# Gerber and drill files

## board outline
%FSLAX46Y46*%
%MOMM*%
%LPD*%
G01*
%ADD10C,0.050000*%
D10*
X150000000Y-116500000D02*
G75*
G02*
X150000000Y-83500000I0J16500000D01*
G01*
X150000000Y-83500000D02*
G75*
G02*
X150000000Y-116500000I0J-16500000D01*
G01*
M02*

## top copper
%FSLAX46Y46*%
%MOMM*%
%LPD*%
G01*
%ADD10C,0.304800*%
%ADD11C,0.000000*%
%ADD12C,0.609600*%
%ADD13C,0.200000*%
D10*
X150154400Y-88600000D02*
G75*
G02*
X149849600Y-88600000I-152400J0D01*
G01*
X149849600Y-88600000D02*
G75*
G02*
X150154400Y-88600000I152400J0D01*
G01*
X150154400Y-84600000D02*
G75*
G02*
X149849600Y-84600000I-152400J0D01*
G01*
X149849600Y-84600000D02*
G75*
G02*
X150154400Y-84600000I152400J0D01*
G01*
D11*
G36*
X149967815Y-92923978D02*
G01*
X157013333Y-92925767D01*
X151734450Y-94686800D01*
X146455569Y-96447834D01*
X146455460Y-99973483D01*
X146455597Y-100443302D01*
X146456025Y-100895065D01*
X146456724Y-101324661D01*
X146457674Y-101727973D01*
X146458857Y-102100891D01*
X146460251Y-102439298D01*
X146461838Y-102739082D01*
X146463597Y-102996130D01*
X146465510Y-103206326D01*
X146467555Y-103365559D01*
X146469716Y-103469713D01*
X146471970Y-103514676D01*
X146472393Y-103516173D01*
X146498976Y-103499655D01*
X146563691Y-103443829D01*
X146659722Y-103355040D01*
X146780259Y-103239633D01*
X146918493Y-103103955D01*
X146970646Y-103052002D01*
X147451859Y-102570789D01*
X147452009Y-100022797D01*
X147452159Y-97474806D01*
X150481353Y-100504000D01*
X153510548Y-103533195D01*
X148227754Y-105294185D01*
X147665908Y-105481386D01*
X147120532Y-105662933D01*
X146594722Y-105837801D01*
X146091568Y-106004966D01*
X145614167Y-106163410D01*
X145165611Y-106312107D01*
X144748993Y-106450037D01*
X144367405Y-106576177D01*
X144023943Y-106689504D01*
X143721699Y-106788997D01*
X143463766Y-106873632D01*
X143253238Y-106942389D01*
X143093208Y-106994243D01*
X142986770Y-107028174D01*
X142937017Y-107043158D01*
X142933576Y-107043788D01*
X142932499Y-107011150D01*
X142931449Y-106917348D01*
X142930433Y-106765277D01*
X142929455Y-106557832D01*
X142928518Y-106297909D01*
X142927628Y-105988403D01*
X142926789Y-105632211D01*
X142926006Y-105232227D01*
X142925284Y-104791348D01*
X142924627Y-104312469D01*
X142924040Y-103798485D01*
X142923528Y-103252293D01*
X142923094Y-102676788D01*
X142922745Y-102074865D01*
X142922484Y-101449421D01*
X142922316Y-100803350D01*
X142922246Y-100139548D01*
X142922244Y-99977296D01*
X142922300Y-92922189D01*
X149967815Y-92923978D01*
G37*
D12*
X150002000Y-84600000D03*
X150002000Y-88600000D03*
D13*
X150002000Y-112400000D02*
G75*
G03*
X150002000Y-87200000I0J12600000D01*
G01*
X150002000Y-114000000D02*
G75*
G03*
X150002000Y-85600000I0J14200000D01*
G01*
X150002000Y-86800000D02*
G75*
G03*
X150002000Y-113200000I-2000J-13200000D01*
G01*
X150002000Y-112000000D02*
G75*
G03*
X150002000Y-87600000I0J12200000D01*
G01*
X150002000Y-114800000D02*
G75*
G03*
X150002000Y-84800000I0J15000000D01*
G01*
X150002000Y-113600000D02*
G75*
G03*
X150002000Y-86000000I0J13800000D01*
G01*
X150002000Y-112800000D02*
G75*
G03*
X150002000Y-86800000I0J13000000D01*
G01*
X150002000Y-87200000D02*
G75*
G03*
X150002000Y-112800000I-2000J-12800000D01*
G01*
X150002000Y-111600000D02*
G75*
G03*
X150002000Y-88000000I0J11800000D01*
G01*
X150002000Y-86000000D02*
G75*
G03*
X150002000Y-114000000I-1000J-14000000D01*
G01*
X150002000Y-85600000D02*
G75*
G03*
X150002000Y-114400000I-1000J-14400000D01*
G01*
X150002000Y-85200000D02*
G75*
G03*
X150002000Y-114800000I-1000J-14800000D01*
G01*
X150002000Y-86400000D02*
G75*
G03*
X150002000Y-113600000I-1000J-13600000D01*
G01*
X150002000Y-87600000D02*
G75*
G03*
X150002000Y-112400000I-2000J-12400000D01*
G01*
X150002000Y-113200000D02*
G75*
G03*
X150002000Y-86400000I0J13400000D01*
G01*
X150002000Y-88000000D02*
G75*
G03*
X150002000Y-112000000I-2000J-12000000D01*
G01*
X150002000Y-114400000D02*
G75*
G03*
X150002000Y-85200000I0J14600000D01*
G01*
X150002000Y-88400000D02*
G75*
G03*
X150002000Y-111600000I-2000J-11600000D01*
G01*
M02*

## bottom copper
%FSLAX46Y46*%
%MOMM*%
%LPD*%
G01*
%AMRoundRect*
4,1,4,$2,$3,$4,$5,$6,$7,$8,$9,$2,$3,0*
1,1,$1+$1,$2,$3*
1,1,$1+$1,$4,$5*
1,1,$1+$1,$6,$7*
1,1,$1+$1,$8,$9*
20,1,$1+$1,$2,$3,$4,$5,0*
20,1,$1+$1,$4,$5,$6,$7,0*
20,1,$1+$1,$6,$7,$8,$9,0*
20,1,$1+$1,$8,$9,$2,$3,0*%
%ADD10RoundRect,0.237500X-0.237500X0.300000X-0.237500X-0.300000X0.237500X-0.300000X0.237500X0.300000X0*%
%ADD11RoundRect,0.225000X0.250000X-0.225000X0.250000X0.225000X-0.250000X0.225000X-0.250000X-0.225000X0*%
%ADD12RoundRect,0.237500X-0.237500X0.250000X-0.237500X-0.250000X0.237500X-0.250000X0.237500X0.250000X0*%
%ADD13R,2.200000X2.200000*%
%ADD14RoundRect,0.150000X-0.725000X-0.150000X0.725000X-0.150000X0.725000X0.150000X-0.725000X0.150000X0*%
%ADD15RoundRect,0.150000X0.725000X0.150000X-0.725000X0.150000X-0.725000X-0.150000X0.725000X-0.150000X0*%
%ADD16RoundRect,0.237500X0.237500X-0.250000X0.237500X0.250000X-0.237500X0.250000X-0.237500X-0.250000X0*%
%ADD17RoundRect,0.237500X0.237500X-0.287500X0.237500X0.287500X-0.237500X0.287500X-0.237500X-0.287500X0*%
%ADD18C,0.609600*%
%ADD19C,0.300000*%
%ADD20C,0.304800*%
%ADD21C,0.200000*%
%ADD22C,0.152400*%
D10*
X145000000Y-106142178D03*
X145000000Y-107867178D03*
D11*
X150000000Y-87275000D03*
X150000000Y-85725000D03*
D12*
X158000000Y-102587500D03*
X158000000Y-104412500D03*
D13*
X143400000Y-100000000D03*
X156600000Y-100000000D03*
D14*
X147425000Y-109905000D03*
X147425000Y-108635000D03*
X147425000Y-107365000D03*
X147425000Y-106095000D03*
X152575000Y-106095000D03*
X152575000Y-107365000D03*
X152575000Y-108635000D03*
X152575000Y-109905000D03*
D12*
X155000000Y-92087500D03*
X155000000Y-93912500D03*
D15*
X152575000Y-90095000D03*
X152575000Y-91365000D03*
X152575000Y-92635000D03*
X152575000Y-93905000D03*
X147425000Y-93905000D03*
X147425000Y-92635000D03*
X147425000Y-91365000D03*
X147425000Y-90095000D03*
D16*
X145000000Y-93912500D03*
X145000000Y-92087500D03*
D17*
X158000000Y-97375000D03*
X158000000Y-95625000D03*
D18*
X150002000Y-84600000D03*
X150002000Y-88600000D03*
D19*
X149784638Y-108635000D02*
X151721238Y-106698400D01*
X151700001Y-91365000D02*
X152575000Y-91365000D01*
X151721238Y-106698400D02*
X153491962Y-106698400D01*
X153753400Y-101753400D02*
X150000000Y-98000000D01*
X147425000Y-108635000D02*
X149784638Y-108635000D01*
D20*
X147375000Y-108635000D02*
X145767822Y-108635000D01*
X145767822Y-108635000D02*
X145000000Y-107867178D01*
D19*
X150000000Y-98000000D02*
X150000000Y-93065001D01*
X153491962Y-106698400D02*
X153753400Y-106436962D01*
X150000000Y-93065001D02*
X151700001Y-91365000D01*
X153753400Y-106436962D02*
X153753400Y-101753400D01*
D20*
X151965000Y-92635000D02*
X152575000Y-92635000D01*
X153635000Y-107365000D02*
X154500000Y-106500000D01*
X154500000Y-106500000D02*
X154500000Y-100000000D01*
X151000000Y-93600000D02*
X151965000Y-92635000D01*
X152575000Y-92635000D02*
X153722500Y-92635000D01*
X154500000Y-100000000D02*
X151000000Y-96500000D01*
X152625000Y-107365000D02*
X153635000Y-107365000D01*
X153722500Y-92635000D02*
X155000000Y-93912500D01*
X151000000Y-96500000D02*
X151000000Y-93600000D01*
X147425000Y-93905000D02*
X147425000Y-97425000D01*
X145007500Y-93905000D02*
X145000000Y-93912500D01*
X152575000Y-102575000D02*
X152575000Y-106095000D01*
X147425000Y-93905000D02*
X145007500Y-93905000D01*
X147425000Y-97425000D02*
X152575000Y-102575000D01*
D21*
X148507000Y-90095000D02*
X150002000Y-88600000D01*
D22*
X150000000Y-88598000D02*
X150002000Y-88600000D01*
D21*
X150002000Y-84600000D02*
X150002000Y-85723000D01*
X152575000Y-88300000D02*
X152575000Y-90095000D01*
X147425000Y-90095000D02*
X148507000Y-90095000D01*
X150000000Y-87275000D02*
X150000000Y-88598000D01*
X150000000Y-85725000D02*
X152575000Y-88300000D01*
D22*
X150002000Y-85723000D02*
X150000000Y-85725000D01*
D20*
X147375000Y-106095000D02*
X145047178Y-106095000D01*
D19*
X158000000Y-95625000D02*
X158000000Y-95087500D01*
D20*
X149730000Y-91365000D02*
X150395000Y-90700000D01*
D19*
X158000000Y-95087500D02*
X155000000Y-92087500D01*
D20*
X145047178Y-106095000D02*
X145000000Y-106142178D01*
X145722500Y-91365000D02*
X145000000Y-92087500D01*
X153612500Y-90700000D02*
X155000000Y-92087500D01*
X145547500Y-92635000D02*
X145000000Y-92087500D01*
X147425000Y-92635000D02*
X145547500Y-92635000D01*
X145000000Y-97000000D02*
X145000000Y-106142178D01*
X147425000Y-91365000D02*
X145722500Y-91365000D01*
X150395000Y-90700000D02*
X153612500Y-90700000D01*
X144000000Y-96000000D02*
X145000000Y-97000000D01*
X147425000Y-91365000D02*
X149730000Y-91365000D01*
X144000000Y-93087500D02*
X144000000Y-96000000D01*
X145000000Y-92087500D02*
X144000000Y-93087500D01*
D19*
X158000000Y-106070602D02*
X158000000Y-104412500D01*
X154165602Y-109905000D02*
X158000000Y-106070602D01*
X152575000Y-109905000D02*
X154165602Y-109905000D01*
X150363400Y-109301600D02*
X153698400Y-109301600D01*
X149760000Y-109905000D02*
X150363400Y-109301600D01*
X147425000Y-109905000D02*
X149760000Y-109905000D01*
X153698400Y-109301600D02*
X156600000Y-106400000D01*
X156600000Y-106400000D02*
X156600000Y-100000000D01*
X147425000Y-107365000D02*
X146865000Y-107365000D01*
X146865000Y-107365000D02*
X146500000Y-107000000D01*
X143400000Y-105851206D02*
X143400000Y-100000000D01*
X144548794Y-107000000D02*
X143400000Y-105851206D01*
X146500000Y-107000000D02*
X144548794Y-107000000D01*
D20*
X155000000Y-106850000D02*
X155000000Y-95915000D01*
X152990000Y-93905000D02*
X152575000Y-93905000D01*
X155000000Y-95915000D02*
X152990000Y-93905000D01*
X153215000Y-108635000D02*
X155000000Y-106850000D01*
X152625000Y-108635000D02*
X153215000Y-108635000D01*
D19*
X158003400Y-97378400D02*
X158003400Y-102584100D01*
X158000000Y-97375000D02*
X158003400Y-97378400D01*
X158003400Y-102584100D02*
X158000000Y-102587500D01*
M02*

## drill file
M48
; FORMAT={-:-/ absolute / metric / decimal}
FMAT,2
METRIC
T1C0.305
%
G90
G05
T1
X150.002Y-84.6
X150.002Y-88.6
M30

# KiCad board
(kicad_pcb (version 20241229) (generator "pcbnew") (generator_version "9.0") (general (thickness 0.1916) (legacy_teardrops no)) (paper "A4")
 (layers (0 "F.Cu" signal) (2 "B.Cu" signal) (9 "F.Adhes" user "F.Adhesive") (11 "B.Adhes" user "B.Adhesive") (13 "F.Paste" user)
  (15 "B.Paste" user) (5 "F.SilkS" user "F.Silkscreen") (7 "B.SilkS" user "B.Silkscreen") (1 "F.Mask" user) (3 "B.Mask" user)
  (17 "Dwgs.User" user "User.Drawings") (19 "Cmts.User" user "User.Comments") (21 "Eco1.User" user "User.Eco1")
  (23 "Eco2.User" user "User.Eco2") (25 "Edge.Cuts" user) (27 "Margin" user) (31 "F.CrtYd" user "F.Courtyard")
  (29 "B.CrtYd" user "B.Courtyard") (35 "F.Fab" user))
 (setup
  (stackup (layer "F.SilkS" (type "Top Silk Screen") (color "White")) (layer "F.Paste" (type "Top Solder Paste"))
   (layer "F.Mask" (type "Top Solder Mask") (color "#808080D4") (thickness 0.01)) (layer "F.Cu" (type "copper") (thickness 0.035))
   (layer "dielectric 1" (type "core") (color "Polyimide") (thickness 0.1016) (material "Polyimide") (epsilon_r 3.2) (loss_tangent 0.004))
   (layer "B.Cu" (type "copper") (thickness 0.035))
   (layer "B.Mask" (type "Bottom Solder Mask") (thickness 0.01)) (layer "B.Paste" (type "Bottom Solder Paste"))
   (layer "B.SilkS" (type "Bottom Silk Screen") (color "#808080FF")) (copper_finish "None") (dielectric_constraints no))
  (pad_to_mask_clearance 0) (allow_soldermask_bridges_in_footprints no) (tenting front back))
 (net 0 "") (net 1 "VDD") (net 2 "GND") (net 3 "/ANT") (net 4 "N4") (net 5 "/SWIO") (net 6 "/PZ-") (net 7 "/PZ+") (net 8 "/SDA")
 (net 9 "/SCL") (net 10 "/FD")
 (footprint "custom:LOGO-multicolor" (layer "F.Cu") (at 150 100 -45)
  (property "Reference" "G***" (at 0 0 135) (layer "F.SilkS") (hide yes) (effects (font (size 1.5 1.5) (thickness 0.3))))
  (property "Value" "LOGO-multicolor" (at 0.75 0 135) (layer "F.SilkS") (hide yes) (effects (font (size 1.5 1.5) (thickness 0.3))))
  (fp_poly
   (pts (xy -2.530558 -4.983441) (xy -5.018052 -0.005469) (xy -2.525119 2.487618) (xy -2.19281 2.819733) (xy -1.873062 3.138875)
    (xy -1.568798 3.442151) (xy -1.282941 3.726664) (xy -1.018412 3.989521) (xy -0.778136 4.227825) (xy -0.565035 4.438682)
    (xy -0.382031 4.619198) (xy -0.232047 4.766477) (xy -0.118006 4.877625) (xy -0.04283 4.949745) (xy -0.009443 4.979945)
    (xy -0.008085 4.980705) (xy -0.000968 4.950228) (xy 0.005317 4.864992) (xy 0.010438 4.734305) (xy 0.014066 4.567467)
    (xy 0.015873 4.373782) (xy 0.016015 4.300168) (xy 0.016015 3.61963) (xy -1.785582 1.817822) (xy -3.587177 0.016014)
    (xy 0.69675 0.016014) (xy 4.980678 0.016014) (xy 2.490387 4.996721) (xy 2.225473 5.526377) (xy 1.968207 6.04039) (xy 1.720054 6.535844)
    (xy 1.482473 7.009831) (xy 1.256937 7.459441) (xy 1.044904 7.881763) (xy 0.847842 8.273888) (xy 0.667213 8.632905)
    (xy 0.504483 8.955904) (xy 0.361117 9.239975) (xy 0.238576 9.482207) (xy 0.138329 9.679692) (xy 0.061837 9.829516)
    (xy 0.010567 9.928772) (xy -0.014018 9.974548) (xy -0.016006 9.977427) (xy -0.039846 9.95511) (xy -0.106917 9.889524)
    (xy -0.215166 9.782712) (xy -0.362543 9.636718) (xy -0.546999 9.453587) (xy -0.766482 9.235363) (xy -1.018941 8.98409)
    (xy -1.302326 8.701812) (xy -1.614585 8.390574) (xy -1.953668 8.05242) (xy -2.317525 7.689394) (xy -2.704103 7.30354)
    (xy -3.111353 6.896903) (xy -3.537224 6.471526) (xy -3.979664 6.029455) (xy -4.436624 5.572733) (xy -4.906053 5.103403)
    (xy -5.020783 4.988675) (xy -10.009458 -0.000078) (xy -5.026261 -4.980745) (xy -0.043063 -9.961413))
   (stroke (width 0) (type solid)) (fill yes) (layer "F.Cu")))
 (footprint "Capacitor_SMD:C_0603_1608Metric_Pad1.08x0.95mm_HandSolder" (layer "B.Cu") (at 145 107.004678 -90)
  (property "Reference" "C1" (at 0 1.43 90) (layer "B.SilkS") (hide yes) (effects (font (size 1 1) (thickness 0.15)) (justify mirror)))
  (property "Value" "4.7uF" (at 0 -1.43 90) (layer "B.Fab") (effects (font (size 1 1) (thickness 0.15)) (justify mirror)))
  (pad "1" smd roundrect (at -0.8625 0 270) (size 1.075 0.95) (layers "B.Cu" "B.Mask" "B.Paste") (roundrect_rratio 0.25) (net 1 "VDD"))
  (pad "2" smd roundrect (at 0.8625 0 270) (size 1.075 0.95) (layers "B.Cu" "B.Mask" "B.Paste") (roundrect_rratio 0.25) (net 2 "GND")))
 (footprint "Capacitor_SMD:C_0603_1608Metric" (layer "B.Cu") (at 150 86.5 90)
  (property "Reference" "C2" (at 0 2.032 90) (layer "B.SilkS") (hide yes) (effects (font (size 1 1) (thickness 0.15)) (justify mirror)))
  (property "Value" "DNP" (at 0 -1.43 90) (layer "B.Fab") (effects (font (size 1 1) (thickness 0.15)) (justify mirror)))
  (pad "1" smd roundrect (at -0.775 0 90) (size 0.9 0.95) (layers "B.Cu" "B.Mask" "B.Paste") (roundrect_rratio 0.25) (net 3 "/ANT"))
  (pad "2" smd roundrect (at 0.775 0 90) (size 0.9 0.95) (layers "B.Cu" "B.Mask" "B.Paste") (roundrect_rratio 0.25) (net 3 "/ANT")))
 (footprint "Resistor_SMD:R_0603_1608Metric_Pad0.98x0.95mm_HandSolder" (layer "B.Cu") (at 158 103.5 -90)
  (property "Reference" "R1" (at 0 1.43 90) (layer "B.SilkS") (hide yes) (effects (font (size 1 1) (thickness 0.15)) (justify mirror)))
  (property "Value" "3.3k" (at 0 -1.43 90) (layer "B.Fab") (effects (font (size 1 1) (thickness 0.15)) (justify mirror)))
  (pad "1" smd roundrect (at -0.9125 0 270) (size 0.975 0.95) (layers "B.Cu" "B.Mask" "B.Paste") (roundrect_rratio 0.25) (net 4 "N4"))
  (pad "2" smd roundrect (at 0.9125 0 270) (size 0.975 0.95) (layers "B.Cu" "B.Mask" "B.Paste") (roundrect_rratio 0.25) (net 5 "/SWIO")))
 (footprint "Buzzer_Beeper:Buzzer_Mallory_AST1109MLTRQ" (layer "B.Cu") (at 150 100)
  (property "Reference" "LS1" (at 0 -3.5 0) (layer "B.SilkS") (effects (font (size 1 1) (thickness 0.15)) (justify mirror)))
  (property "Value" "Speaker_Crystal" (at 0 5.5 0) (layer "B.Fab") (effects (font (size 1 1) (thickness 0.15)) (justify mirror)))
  (pad "1" smd rect (at -6.6 0) (size 2.2 2.2) (layers "B.Cu" "B.Mask" "B.Paste") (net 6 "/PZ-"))
  (pad "2" smd rect (at 6.6 0) (size 2.2 2.2) (layers "B.Cu" "B.Mask" "B.Paste") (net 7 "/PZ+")))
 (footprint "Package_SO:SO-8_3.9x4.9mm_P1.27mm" (layer "B.Cu") (at 150 108)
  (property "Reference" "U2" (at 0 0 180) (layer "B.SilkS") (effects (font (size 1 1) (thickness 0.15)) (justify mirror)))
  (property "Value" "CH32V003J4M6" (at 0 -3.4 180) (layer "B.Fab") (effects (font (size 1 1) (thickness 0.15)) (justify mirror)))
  (pad "1" smd roundrect (at -2.575 1.905) (size 1.75 0.6) (layers "B.Cu" "B.Mask" "B.Paste") (roundrect_rratio 0.25) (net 7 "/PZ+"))
  (pad "2" smd roundrect (at -2.575 0.635) (size 1.75 0.6) (layers "B.Cu" "B.Mask" "B.Paste") (roundrect_rratio 0.25) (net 2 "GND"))
  (pad "3" smd roundrect (at -2.575 -0.635) (size 1.75 0.6) (layers "B.Cu" "B.Mask" "B.Paste") (roundrect_rratio 0.25) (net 6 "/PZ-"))
  (pad "4" smd roundrect (at -2.575 -1.905) (size 1.75 0.6) (layers "B.Cu" "B.Mask" "B.Paste") (roundrect_rratio 0.25) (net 1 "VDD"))
  (pad "5" smd roundrect (at 2.575 -1.905) (size 1.75 0.6) (layers "B.Cu" "B.Mask" "B.Paste") (roundrect_rratio 0.25) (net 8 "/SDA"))
  (pad "6" smd roundrect (at 2.575 -0.635) (size 1.75 0.6) (layers "B.Cu" "B.Mask" "B.Paste") (roundrect_rratio 0.25) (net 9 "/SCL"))
  (pad "7" smd roundrect (at 2.575 0.635) (size 1.75 0.6) (layers "B.Cu" "B.Mask" "B.Paste") (roundrect_rratio 0.25) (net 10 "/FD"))
  (pad "8" smd roundrect (at 2.575 1.905) (size 1.75 0.6) (layers "B.Cu" "B.Mask" "B.Paste") (roundrect_rratio 0.25) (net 5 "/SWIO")))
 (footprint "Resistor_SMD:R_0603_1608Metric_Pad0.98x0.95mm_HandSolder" (layer "B.Cu") (at 155 93 -90)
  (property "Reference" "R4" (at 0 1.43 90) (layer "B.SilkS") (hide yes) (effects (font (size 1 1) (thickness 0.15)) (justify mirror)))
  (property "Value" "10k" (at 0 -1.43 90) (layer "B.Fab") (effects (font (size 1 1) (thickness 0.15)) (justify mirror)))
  (pad "1" smd roundrect (at -0.9125 0 270) (size 0.975 0.95) (layers "B.Cu" "B.Mask" "B.Paste") (roundrect_rratio 0.25) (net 1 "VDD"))
  (pad "2" smd roundrect (at 0.9125 0 270) (size 0.975 0.95) (layers "B.Cu" "B.Mask" "B.Paste") (roundrect_rratio 0.25) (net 9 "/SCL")))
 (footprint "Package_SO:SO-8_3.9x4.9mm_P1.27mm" (layer "B.Cu") (at 150 92 180)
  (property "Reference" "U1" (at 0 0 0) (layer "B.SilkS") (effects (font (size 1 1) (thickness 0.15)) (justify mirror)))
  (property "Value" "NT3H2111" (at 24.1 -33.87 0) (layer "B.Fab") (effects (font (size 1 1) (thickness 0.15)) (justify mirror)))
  (pad "1" smd roundrect (at -2.575 1.905 180) (size 1.75 0.6) (layers "B.Cu" "B.Mask" "B.Paste") (roundrect_rratio 0.25) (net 3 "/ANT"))
  (pad "2" smd roundrect (at -2.575 0.635 180) (size 1.75 0.6) (layers "B.Cu" "B.Mask" "B.Paste") (roundrect_rratio 0.25) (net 2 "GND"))
  (pad "3" smd roundrect (at -2.575 -0.635 180) (size 1.75 0.6) (layers "B.Cu" "B.Mask" "B.Paste") (roundrect_rratio 0.25) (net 9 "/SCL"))
  (pad "4" smd roundrect (at -2.575 -1.905 180) (size 1.75 0.6) (layers "B.Cu" "B.Mask" "B.Paste") (roundrect_rratio 0.25) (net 10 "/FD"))
  (pad "5" smd roundrect (at 2.575 -1.905 180) (size 1.75 0.6) (layers "B.Cu" "B.Mask" "B.Paste") (roundrect_rratio 0.25) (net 8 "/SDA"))
  (pad "6" smd roundrect (at 2.575 -0.635 180) (size 1.75 0.6) (layers "B.Cu" "B.Mask" "B.Paste") (roundrect_rratio 0.25) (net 1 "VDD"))
  (pad "7" smd roundrect (at 2.575 0.635 180) (size 1.75 0.6) (layers "B.Cu" "B.Mask" "B.Paste") (roundrect_rratio 0.25) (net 1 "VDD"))
  (pad "8" smd roundrect (at 2.575 1.905 180) (size 1.75 0.6) (layers "B.Cu" "B.Mask" "B.Paste") (roundrect_rratio 0.25) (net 3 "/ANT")))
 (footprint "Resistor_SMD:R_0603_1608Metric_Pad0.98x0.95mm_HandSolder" (layer "B.Cu") (at 145 93 90)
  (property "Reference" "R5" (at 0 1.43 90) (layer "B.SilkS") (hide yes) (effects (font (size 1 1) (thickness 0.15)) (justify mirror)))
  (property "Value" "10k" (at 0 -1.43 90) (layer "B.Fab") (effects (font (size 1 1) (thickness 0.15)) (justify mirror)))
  (pad "1" smd roundrect (at -0.9125 0 90) (size 0.975 0.95) (layers "B.Cu" "B.Mask" "B.Paste") (roundrect_rratio 0.25) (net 8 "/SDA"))
  (pad "2" smd roundrect (at 0.9125 0 90) (size 0.975 0.95) (layers "B.Cu" "B.Mask" "B.Paste") (roundrect_rratio 0.25) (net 1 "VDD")))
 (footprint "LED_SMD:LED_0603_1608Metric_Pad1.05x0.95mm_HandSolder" (layer "B.Cu") (at 158 96.5 90)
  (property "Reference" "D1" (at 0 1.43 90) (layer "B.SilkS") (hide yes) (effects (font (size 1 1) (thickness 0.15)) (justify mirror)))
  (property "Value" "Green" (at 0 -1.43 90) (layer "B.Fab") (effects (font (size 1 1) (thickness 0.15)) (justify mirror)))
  (pad "1" smd roundrect (at -0.875 0 90) (size 1.05 0.95) (layers "B.Cu" "B.Mask" "B.Paste") (roundrect_rratio 0.25) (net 4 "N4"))
  (pad "2" smd roundrect (at 0.875 0 90) (size 1.05 0.95) (layers "B.Cu" "B.Mask" "B.Paste") (roundrect_rratio 0.25) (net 1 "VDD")))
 (gr_circle (center 150.002 88.6) (end 150.3068 88.6) (stroke (width 0) (type solid)) (fill yes) (layer "F.Cu") (net 3))
 (gr_circle (center 150.002 84.6) (end 150.3068 84.6) (stroke (width 0) (type solid)) (fill yes) (layer "F.Cu") (net 3))
 (gr_arc (start 150 116.5) (mid 133.5 100) (end 150 83.5) (stroke (width 0.05) (type solid)) (layer "Edge.Cuts"))
 (gr_arc (start 150 83.5) (mid 166.5 100) (end 150 116.5) (stroke (width 0.05) (type solid)) (layer "Edge.Cuts"))
 (segment (start 149.784638 108.635) (end 151.721238 106.6984) (width 0.3) (layer "B.Cu") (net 2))
 (segment (start 151.700001 91.365) (end 152.575 91.365) (width 0.3) (layer "B.Cu") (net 2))
 (segment (start 151.721238 106.6984) (end 153.491962 106.6984) (width 0.3) (layer "B.Cu") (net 2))
 (segment (start 153.7534 101.7534) (end 150 98) (width 0.3) (layer "B.Cu") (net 2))
 (segment (start 147.425 108.635) (end 149.784638 108.635) (width 0.3) (layer "B.Cu") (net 2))
 (segment (start 147.375 108.635) (end 145.767822 108.635) (width 0.3048) (layer "B.Cu") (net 2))
 (segment (start 145.767822 108.635) (end 145 107.867178) (width 0.3048) (layer "B.Cu") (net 2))
 (segment (start 150 98) (end 150 93.065001) (width 0.3) (layer "B.Cu") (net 2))
 (segment (start 153.491962 106.6984) (end 153.7534 106.436962) (width 0.3) (layer "B.Cu") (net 2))
 (segment (start 150 93.065001) (end 151.700001 91.365) (width 0.3) (layer "B.Cu") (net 2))
 (segment (start 153.7534 106.436962) (end 153.7534 101.7534) (width 0.3) (layer "B.Cu") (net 2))
 (segment (start 151.965 92.635) (end 152.575 92.635) (width 0.3048) (layer "B.Cu") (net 9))
 (segment (start 153.635 107.365) (end 154.5 106.5) (width 0.3048) (layer "B.Cu") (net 9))
 (segment (start 154.5 106.5) (end 154.5 100) (width 0.3048) (layer "B.Cu") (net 9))
 (segment (start 151 93.6) (end 151.965 92.635) (width 0.3048) (layer "B.Cu") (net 9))
 (segment (start 152.575 92.635) (end 153.7225 92.635) (width 0.3048) (layer "B.Cu") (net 9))
 (segment (start 154.5 100) (end 151 96.5) (width 0.3048) (layer "B.Cu") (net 9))
 (segment (start 152.625 107.365) (end 153.635 107.365) (width 0.3048) (layer "B.Cu") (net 9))
 (segment (start 153.7225 92.635) (end 155 93.9125) (width 0.3048) (layer "B.Cu") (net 9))
 (segment (start 151 96.5) (end 151 93.6) (width 0.3048) (layer "B.Cu") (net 9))
 (segment (start 147.425 93.905) (end 147.425 97.425) (width 0.3048) (layer "B.Cu") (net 8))
 (segment (start 145.0075 93.905) (end 145 93.9125) (width 0.3048) (layer "B.Cu") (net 8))
 (segment (start 152.575 102.575) (end 152.575 106.095) (width 0.3048) (layer "B.Cu") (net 8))
 (segment (start 147.425 93.905) (end 145.0075 93.905) (width 0.3048) (layer "B.Cu") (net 8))
 (segment (start 147.425 97.425) (end 152.575 102.575) (width 0.3048) (layer "B.Cu") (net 8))
 (via (at 150.002 84.6) (size 0.6096) (drill 0.3048) (layers "F.Cu" "B.Cu") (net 3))
 (via (at 150.002 88.6) (size 0.6096) (drill 0.3048) (layers "F.Cu" "B.Cu") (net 3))
 (arc (start 150.002 112.4) (mid 162.602 99.8) (end 150.002 87.2) (width 0.2) (layer "F.Cu") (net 3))
 (arc (start 150.002 114) (mid 164.202 99.8) (end 150.002 85.6) (width 0.2) (layer "F.Cu") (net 3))
 (arc (start 150.002 86.8) (mid 136.8 100) (end 150.002 113.2) (width 0.2) (layer "F.Cu") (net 3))
 (arc (start 150.002 112) (mid 162.202 99.8) (end 150.002 87.6) (width 0.2) (layer "F.Cu") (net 3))
 (arc (start 150.002 114.8) (mid 165.002 99.8) (end 150.002 84.8) (width 0.2) (layer "F.Cu") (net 3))
 (arc (start 150.002 113.6) (mid 163.802 99.8) (end 150.002 86) (width 0.2) (layer "F.Cu") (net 3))
 (arc (start 150.002 112.8) (mid 163.002 99.8) (end 150.002 86.8) (width 0.2) (layer "F.Cu") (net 3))
 (arc (start 150.002 87.2) (mid 137.2 100) (end 150.002 112.8) (width 0.2) (layer "F.Cu") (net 3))
 (arc (start 150.002 111.6) (mid 161.802 99.8) (end 150.002 88) (width 0.2) (layer "F.Cu") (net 3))
 (arc (start 150.002 86) (mid 136.001 100) (end 150.002 114) (width 0.2) (layer "F.Cu") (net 3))
 (arc (start 150.002 85.6) (mid 135.601 100) (end 150.002 114.4) (width 0.2) (layer "F.Cu") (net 3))
 (arc (start 150.002 85.2) (mid 135.201 100) (end 150.002 114.8) (width 0.2) (layer "F.Cu") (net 3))
 (arc (start 150.002 86.4) (mid 136.401 100) (end 150.002 113.6) (width 0.2) (layer "F.Cu") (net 3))
 (arc (start 150.002 87.6) (mid 137.6 100) (end 150.002 112.4) (width 0.2) (layer "F.Cu") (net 3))
 (arc (start 150.002 113.2) (mid 163.402 99.8) (end 150.002 86.4) (width 0.2) (layer "F.Cu") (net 3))
 (arc (start 150.002 88) (mid 138 100) (end 150.002 112) (width 0.2) (layer "F.Cu") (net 3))
 (arc (start 150.002 114.4) (mid 164.602 99.8) (end 150.002 85.2) (width 0.2) (layer "F.Cu") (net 3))
 (arc (start 150.002 88.4) (mid 138.4 100) (end 150.002 111.6) (width 0.2) (layer "F.Cu") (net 3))
 (segment (start 148.507 90.095) (end 150.002 88.6) (width 0.2) (layer "B.Cu") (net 3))
 (segment (start 150 88.598) (end 150.002 88.6) (width 0.1524) (layer "B.Cu") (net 3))
 (segment (start 150.002 84.6) (end 150.002 85.723) (width 0.2) (layer "B.Cu") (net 3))
 (segment (start 152.575 88.3) (end 152.575 90.095) (width 0.2) (layer "B.Cu") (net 3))
 (segment (start 147.425 90.095) (end 148.507 90.095) (width 0.2) (layer "B.Cu") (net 3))
 (segment (start 150 87.275) (end 150 88.598) (width 0.2) (layer "B.Cu") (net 3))
 (segment (start 150 85.725) (end 152.575 88.3) (width 0.2) (layer "B.Cu") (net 3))
 (segment (start 150.002 85.723) (end 150 85.725) (width 0.1524) (layer "B.Cu") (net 3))
 (segment (start 147.375 106.095) (end 145.047178 106.095) (width 0.3048) (layer "B.Cu") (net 1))
 (segment (start 158 95.625) (end 158 95.0875) (width 0.3) (layer "B.Cu") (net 1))
 (segment (start 149.73 91.365) (end 150.395 90.7) (width 0.3048) (layer "B.Cu") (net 1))
 (segment (start 158 95.0875) (end 155 92.0875) (width 0.3) (layer "B.Cu") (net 1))
 (segment (start 145.047178 106.095) (end 145 106.142178) (width 0.3048) (layer "B.Cu") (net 1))
 (segment (start 145.7225 91.365) (end 145 92.0875) (width 0.3048) (layer "B.Cu") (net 1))
 (segment (start 153.6125 90.7) (end 155 92.0875) (width 0.3048) (layer "B.Cu") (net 1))
 (segment (start 145.5475 92.635) (end 145 92.0875) (width 0.3048) (layer "B.Cu") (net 1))
 (segment (start 147.425 92.635) (end 145.5475 92.635) (width 0.3048) (layer "B.Cu") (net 1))
 (segment (start 145 97) (end 145 106.142178) (width 0.3048) (layer "B.Cu") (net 1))
 (segment (start 147.425 91.365) (end 145.7225 91.365) (width 0.3048) (layer "B.Cu") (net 1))
 (segment (start 150.395 90.7) (end 153.6125 90.7) (width 0.3048) (layer "B.Cu") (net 1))
 (segment (start 144 96) (end 145 97) (width 0.3048) (layer "B.Cu") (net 1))
 (segment (start 147.425 91.365) (end 149.73 91.365) (width 0.3048) (layer "B.Cu") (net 1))
 (segment (start 144 93.0875) (end 144 96) (width 0.3048) (layer "B.Cu") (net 1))
 (segment (start 145 92.0875) (end 144 93.0875) (width 0.3048) (layer "B.Cu") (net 1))
 (segment (start 158 106.070602) (end 158 104.4125) (width 0.3) (layer "B.Cu") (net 5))
 (segment (start 154.165602 109.905) (end 158 106.070602) (width 0.3) (layer "B.Cu") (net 5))
 (segment (start 152.575 109.905) (end 154.165602 109.905) (width 0.3) (layer "B.Cu") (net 5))
 (segment (start 150.3634 109.3016) (end 153.6984 109.3016) (width 0.3) (layer "B.Cu") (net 7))
 (segment (start 149.76 109.905) (end 150.3634 109.3016) (width 0.3) (layer "B.Cu") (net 7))
 (segment (start 147.425 109.905) (end 149.76 109.905) (width 0.3) (layer "B.Cu") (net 7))
 (segment (start 153.6984 109.3016) (end 156.6 106.4) (width 0.3) (layer "B.Cu") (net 7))
 (segment (start 156.6 106.4) (end 156.6 100) (width 0.3) (layer "B.Cu") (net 7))
 (segment (start 147.425 107.365) (end 146.865 107.365) (width 0.3) (layer "B.Cu") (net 6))
 (segment (start 146.865 107.365) (end 146.5 107) (width 0.3) (layer "B.Cu") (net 6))
 (segment (start 143.4 105.851206) (end 143.4 100) (width 0.3) (layer "B.Cu") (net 6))
 (segment (start 144.548794 107) (end 143.4 105.851206) (width 0.3) (layer "B.Cu") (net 6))
 (segment (start 146.5 107) (end 144.548794 107) (width 0.3) (layer "B.Cu") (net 6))
 (segment (start 155 106.85) (end 155 95.915) (width 0.3048) (layer "B.Cu") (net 10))
 (segment (start 152.99 93.905) (end 152.575 93.905) (width 0.3048) (layer "B.Cu") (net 10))
 (segment (start 155 95.915) (end 152.99 93.905) (width 0.3048) (layer "B.Cu") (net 10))
 (segment (start 153.215 108.635) (end 155 106.85) (width 0.3048) (layer "B.Cu") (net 10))
 (segment (start 152.625 108.635) (end 153.215 108.635) (width 0.3048) (layer "B.Cu") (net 10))
 (segment (start 158.0034 97.3784) (end 158.0034 102.5841) (width 0.3) (layer "B.Cu") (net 4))
 (segment (start 158 97.375) (end 158.0034 97.3784) (width 0.3) (layer "B.Cu") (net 4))
 (segment (start 158.0034 102.5841) (end 158 102.5875) (width 0.3) (layer "B.Cu") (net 4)))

